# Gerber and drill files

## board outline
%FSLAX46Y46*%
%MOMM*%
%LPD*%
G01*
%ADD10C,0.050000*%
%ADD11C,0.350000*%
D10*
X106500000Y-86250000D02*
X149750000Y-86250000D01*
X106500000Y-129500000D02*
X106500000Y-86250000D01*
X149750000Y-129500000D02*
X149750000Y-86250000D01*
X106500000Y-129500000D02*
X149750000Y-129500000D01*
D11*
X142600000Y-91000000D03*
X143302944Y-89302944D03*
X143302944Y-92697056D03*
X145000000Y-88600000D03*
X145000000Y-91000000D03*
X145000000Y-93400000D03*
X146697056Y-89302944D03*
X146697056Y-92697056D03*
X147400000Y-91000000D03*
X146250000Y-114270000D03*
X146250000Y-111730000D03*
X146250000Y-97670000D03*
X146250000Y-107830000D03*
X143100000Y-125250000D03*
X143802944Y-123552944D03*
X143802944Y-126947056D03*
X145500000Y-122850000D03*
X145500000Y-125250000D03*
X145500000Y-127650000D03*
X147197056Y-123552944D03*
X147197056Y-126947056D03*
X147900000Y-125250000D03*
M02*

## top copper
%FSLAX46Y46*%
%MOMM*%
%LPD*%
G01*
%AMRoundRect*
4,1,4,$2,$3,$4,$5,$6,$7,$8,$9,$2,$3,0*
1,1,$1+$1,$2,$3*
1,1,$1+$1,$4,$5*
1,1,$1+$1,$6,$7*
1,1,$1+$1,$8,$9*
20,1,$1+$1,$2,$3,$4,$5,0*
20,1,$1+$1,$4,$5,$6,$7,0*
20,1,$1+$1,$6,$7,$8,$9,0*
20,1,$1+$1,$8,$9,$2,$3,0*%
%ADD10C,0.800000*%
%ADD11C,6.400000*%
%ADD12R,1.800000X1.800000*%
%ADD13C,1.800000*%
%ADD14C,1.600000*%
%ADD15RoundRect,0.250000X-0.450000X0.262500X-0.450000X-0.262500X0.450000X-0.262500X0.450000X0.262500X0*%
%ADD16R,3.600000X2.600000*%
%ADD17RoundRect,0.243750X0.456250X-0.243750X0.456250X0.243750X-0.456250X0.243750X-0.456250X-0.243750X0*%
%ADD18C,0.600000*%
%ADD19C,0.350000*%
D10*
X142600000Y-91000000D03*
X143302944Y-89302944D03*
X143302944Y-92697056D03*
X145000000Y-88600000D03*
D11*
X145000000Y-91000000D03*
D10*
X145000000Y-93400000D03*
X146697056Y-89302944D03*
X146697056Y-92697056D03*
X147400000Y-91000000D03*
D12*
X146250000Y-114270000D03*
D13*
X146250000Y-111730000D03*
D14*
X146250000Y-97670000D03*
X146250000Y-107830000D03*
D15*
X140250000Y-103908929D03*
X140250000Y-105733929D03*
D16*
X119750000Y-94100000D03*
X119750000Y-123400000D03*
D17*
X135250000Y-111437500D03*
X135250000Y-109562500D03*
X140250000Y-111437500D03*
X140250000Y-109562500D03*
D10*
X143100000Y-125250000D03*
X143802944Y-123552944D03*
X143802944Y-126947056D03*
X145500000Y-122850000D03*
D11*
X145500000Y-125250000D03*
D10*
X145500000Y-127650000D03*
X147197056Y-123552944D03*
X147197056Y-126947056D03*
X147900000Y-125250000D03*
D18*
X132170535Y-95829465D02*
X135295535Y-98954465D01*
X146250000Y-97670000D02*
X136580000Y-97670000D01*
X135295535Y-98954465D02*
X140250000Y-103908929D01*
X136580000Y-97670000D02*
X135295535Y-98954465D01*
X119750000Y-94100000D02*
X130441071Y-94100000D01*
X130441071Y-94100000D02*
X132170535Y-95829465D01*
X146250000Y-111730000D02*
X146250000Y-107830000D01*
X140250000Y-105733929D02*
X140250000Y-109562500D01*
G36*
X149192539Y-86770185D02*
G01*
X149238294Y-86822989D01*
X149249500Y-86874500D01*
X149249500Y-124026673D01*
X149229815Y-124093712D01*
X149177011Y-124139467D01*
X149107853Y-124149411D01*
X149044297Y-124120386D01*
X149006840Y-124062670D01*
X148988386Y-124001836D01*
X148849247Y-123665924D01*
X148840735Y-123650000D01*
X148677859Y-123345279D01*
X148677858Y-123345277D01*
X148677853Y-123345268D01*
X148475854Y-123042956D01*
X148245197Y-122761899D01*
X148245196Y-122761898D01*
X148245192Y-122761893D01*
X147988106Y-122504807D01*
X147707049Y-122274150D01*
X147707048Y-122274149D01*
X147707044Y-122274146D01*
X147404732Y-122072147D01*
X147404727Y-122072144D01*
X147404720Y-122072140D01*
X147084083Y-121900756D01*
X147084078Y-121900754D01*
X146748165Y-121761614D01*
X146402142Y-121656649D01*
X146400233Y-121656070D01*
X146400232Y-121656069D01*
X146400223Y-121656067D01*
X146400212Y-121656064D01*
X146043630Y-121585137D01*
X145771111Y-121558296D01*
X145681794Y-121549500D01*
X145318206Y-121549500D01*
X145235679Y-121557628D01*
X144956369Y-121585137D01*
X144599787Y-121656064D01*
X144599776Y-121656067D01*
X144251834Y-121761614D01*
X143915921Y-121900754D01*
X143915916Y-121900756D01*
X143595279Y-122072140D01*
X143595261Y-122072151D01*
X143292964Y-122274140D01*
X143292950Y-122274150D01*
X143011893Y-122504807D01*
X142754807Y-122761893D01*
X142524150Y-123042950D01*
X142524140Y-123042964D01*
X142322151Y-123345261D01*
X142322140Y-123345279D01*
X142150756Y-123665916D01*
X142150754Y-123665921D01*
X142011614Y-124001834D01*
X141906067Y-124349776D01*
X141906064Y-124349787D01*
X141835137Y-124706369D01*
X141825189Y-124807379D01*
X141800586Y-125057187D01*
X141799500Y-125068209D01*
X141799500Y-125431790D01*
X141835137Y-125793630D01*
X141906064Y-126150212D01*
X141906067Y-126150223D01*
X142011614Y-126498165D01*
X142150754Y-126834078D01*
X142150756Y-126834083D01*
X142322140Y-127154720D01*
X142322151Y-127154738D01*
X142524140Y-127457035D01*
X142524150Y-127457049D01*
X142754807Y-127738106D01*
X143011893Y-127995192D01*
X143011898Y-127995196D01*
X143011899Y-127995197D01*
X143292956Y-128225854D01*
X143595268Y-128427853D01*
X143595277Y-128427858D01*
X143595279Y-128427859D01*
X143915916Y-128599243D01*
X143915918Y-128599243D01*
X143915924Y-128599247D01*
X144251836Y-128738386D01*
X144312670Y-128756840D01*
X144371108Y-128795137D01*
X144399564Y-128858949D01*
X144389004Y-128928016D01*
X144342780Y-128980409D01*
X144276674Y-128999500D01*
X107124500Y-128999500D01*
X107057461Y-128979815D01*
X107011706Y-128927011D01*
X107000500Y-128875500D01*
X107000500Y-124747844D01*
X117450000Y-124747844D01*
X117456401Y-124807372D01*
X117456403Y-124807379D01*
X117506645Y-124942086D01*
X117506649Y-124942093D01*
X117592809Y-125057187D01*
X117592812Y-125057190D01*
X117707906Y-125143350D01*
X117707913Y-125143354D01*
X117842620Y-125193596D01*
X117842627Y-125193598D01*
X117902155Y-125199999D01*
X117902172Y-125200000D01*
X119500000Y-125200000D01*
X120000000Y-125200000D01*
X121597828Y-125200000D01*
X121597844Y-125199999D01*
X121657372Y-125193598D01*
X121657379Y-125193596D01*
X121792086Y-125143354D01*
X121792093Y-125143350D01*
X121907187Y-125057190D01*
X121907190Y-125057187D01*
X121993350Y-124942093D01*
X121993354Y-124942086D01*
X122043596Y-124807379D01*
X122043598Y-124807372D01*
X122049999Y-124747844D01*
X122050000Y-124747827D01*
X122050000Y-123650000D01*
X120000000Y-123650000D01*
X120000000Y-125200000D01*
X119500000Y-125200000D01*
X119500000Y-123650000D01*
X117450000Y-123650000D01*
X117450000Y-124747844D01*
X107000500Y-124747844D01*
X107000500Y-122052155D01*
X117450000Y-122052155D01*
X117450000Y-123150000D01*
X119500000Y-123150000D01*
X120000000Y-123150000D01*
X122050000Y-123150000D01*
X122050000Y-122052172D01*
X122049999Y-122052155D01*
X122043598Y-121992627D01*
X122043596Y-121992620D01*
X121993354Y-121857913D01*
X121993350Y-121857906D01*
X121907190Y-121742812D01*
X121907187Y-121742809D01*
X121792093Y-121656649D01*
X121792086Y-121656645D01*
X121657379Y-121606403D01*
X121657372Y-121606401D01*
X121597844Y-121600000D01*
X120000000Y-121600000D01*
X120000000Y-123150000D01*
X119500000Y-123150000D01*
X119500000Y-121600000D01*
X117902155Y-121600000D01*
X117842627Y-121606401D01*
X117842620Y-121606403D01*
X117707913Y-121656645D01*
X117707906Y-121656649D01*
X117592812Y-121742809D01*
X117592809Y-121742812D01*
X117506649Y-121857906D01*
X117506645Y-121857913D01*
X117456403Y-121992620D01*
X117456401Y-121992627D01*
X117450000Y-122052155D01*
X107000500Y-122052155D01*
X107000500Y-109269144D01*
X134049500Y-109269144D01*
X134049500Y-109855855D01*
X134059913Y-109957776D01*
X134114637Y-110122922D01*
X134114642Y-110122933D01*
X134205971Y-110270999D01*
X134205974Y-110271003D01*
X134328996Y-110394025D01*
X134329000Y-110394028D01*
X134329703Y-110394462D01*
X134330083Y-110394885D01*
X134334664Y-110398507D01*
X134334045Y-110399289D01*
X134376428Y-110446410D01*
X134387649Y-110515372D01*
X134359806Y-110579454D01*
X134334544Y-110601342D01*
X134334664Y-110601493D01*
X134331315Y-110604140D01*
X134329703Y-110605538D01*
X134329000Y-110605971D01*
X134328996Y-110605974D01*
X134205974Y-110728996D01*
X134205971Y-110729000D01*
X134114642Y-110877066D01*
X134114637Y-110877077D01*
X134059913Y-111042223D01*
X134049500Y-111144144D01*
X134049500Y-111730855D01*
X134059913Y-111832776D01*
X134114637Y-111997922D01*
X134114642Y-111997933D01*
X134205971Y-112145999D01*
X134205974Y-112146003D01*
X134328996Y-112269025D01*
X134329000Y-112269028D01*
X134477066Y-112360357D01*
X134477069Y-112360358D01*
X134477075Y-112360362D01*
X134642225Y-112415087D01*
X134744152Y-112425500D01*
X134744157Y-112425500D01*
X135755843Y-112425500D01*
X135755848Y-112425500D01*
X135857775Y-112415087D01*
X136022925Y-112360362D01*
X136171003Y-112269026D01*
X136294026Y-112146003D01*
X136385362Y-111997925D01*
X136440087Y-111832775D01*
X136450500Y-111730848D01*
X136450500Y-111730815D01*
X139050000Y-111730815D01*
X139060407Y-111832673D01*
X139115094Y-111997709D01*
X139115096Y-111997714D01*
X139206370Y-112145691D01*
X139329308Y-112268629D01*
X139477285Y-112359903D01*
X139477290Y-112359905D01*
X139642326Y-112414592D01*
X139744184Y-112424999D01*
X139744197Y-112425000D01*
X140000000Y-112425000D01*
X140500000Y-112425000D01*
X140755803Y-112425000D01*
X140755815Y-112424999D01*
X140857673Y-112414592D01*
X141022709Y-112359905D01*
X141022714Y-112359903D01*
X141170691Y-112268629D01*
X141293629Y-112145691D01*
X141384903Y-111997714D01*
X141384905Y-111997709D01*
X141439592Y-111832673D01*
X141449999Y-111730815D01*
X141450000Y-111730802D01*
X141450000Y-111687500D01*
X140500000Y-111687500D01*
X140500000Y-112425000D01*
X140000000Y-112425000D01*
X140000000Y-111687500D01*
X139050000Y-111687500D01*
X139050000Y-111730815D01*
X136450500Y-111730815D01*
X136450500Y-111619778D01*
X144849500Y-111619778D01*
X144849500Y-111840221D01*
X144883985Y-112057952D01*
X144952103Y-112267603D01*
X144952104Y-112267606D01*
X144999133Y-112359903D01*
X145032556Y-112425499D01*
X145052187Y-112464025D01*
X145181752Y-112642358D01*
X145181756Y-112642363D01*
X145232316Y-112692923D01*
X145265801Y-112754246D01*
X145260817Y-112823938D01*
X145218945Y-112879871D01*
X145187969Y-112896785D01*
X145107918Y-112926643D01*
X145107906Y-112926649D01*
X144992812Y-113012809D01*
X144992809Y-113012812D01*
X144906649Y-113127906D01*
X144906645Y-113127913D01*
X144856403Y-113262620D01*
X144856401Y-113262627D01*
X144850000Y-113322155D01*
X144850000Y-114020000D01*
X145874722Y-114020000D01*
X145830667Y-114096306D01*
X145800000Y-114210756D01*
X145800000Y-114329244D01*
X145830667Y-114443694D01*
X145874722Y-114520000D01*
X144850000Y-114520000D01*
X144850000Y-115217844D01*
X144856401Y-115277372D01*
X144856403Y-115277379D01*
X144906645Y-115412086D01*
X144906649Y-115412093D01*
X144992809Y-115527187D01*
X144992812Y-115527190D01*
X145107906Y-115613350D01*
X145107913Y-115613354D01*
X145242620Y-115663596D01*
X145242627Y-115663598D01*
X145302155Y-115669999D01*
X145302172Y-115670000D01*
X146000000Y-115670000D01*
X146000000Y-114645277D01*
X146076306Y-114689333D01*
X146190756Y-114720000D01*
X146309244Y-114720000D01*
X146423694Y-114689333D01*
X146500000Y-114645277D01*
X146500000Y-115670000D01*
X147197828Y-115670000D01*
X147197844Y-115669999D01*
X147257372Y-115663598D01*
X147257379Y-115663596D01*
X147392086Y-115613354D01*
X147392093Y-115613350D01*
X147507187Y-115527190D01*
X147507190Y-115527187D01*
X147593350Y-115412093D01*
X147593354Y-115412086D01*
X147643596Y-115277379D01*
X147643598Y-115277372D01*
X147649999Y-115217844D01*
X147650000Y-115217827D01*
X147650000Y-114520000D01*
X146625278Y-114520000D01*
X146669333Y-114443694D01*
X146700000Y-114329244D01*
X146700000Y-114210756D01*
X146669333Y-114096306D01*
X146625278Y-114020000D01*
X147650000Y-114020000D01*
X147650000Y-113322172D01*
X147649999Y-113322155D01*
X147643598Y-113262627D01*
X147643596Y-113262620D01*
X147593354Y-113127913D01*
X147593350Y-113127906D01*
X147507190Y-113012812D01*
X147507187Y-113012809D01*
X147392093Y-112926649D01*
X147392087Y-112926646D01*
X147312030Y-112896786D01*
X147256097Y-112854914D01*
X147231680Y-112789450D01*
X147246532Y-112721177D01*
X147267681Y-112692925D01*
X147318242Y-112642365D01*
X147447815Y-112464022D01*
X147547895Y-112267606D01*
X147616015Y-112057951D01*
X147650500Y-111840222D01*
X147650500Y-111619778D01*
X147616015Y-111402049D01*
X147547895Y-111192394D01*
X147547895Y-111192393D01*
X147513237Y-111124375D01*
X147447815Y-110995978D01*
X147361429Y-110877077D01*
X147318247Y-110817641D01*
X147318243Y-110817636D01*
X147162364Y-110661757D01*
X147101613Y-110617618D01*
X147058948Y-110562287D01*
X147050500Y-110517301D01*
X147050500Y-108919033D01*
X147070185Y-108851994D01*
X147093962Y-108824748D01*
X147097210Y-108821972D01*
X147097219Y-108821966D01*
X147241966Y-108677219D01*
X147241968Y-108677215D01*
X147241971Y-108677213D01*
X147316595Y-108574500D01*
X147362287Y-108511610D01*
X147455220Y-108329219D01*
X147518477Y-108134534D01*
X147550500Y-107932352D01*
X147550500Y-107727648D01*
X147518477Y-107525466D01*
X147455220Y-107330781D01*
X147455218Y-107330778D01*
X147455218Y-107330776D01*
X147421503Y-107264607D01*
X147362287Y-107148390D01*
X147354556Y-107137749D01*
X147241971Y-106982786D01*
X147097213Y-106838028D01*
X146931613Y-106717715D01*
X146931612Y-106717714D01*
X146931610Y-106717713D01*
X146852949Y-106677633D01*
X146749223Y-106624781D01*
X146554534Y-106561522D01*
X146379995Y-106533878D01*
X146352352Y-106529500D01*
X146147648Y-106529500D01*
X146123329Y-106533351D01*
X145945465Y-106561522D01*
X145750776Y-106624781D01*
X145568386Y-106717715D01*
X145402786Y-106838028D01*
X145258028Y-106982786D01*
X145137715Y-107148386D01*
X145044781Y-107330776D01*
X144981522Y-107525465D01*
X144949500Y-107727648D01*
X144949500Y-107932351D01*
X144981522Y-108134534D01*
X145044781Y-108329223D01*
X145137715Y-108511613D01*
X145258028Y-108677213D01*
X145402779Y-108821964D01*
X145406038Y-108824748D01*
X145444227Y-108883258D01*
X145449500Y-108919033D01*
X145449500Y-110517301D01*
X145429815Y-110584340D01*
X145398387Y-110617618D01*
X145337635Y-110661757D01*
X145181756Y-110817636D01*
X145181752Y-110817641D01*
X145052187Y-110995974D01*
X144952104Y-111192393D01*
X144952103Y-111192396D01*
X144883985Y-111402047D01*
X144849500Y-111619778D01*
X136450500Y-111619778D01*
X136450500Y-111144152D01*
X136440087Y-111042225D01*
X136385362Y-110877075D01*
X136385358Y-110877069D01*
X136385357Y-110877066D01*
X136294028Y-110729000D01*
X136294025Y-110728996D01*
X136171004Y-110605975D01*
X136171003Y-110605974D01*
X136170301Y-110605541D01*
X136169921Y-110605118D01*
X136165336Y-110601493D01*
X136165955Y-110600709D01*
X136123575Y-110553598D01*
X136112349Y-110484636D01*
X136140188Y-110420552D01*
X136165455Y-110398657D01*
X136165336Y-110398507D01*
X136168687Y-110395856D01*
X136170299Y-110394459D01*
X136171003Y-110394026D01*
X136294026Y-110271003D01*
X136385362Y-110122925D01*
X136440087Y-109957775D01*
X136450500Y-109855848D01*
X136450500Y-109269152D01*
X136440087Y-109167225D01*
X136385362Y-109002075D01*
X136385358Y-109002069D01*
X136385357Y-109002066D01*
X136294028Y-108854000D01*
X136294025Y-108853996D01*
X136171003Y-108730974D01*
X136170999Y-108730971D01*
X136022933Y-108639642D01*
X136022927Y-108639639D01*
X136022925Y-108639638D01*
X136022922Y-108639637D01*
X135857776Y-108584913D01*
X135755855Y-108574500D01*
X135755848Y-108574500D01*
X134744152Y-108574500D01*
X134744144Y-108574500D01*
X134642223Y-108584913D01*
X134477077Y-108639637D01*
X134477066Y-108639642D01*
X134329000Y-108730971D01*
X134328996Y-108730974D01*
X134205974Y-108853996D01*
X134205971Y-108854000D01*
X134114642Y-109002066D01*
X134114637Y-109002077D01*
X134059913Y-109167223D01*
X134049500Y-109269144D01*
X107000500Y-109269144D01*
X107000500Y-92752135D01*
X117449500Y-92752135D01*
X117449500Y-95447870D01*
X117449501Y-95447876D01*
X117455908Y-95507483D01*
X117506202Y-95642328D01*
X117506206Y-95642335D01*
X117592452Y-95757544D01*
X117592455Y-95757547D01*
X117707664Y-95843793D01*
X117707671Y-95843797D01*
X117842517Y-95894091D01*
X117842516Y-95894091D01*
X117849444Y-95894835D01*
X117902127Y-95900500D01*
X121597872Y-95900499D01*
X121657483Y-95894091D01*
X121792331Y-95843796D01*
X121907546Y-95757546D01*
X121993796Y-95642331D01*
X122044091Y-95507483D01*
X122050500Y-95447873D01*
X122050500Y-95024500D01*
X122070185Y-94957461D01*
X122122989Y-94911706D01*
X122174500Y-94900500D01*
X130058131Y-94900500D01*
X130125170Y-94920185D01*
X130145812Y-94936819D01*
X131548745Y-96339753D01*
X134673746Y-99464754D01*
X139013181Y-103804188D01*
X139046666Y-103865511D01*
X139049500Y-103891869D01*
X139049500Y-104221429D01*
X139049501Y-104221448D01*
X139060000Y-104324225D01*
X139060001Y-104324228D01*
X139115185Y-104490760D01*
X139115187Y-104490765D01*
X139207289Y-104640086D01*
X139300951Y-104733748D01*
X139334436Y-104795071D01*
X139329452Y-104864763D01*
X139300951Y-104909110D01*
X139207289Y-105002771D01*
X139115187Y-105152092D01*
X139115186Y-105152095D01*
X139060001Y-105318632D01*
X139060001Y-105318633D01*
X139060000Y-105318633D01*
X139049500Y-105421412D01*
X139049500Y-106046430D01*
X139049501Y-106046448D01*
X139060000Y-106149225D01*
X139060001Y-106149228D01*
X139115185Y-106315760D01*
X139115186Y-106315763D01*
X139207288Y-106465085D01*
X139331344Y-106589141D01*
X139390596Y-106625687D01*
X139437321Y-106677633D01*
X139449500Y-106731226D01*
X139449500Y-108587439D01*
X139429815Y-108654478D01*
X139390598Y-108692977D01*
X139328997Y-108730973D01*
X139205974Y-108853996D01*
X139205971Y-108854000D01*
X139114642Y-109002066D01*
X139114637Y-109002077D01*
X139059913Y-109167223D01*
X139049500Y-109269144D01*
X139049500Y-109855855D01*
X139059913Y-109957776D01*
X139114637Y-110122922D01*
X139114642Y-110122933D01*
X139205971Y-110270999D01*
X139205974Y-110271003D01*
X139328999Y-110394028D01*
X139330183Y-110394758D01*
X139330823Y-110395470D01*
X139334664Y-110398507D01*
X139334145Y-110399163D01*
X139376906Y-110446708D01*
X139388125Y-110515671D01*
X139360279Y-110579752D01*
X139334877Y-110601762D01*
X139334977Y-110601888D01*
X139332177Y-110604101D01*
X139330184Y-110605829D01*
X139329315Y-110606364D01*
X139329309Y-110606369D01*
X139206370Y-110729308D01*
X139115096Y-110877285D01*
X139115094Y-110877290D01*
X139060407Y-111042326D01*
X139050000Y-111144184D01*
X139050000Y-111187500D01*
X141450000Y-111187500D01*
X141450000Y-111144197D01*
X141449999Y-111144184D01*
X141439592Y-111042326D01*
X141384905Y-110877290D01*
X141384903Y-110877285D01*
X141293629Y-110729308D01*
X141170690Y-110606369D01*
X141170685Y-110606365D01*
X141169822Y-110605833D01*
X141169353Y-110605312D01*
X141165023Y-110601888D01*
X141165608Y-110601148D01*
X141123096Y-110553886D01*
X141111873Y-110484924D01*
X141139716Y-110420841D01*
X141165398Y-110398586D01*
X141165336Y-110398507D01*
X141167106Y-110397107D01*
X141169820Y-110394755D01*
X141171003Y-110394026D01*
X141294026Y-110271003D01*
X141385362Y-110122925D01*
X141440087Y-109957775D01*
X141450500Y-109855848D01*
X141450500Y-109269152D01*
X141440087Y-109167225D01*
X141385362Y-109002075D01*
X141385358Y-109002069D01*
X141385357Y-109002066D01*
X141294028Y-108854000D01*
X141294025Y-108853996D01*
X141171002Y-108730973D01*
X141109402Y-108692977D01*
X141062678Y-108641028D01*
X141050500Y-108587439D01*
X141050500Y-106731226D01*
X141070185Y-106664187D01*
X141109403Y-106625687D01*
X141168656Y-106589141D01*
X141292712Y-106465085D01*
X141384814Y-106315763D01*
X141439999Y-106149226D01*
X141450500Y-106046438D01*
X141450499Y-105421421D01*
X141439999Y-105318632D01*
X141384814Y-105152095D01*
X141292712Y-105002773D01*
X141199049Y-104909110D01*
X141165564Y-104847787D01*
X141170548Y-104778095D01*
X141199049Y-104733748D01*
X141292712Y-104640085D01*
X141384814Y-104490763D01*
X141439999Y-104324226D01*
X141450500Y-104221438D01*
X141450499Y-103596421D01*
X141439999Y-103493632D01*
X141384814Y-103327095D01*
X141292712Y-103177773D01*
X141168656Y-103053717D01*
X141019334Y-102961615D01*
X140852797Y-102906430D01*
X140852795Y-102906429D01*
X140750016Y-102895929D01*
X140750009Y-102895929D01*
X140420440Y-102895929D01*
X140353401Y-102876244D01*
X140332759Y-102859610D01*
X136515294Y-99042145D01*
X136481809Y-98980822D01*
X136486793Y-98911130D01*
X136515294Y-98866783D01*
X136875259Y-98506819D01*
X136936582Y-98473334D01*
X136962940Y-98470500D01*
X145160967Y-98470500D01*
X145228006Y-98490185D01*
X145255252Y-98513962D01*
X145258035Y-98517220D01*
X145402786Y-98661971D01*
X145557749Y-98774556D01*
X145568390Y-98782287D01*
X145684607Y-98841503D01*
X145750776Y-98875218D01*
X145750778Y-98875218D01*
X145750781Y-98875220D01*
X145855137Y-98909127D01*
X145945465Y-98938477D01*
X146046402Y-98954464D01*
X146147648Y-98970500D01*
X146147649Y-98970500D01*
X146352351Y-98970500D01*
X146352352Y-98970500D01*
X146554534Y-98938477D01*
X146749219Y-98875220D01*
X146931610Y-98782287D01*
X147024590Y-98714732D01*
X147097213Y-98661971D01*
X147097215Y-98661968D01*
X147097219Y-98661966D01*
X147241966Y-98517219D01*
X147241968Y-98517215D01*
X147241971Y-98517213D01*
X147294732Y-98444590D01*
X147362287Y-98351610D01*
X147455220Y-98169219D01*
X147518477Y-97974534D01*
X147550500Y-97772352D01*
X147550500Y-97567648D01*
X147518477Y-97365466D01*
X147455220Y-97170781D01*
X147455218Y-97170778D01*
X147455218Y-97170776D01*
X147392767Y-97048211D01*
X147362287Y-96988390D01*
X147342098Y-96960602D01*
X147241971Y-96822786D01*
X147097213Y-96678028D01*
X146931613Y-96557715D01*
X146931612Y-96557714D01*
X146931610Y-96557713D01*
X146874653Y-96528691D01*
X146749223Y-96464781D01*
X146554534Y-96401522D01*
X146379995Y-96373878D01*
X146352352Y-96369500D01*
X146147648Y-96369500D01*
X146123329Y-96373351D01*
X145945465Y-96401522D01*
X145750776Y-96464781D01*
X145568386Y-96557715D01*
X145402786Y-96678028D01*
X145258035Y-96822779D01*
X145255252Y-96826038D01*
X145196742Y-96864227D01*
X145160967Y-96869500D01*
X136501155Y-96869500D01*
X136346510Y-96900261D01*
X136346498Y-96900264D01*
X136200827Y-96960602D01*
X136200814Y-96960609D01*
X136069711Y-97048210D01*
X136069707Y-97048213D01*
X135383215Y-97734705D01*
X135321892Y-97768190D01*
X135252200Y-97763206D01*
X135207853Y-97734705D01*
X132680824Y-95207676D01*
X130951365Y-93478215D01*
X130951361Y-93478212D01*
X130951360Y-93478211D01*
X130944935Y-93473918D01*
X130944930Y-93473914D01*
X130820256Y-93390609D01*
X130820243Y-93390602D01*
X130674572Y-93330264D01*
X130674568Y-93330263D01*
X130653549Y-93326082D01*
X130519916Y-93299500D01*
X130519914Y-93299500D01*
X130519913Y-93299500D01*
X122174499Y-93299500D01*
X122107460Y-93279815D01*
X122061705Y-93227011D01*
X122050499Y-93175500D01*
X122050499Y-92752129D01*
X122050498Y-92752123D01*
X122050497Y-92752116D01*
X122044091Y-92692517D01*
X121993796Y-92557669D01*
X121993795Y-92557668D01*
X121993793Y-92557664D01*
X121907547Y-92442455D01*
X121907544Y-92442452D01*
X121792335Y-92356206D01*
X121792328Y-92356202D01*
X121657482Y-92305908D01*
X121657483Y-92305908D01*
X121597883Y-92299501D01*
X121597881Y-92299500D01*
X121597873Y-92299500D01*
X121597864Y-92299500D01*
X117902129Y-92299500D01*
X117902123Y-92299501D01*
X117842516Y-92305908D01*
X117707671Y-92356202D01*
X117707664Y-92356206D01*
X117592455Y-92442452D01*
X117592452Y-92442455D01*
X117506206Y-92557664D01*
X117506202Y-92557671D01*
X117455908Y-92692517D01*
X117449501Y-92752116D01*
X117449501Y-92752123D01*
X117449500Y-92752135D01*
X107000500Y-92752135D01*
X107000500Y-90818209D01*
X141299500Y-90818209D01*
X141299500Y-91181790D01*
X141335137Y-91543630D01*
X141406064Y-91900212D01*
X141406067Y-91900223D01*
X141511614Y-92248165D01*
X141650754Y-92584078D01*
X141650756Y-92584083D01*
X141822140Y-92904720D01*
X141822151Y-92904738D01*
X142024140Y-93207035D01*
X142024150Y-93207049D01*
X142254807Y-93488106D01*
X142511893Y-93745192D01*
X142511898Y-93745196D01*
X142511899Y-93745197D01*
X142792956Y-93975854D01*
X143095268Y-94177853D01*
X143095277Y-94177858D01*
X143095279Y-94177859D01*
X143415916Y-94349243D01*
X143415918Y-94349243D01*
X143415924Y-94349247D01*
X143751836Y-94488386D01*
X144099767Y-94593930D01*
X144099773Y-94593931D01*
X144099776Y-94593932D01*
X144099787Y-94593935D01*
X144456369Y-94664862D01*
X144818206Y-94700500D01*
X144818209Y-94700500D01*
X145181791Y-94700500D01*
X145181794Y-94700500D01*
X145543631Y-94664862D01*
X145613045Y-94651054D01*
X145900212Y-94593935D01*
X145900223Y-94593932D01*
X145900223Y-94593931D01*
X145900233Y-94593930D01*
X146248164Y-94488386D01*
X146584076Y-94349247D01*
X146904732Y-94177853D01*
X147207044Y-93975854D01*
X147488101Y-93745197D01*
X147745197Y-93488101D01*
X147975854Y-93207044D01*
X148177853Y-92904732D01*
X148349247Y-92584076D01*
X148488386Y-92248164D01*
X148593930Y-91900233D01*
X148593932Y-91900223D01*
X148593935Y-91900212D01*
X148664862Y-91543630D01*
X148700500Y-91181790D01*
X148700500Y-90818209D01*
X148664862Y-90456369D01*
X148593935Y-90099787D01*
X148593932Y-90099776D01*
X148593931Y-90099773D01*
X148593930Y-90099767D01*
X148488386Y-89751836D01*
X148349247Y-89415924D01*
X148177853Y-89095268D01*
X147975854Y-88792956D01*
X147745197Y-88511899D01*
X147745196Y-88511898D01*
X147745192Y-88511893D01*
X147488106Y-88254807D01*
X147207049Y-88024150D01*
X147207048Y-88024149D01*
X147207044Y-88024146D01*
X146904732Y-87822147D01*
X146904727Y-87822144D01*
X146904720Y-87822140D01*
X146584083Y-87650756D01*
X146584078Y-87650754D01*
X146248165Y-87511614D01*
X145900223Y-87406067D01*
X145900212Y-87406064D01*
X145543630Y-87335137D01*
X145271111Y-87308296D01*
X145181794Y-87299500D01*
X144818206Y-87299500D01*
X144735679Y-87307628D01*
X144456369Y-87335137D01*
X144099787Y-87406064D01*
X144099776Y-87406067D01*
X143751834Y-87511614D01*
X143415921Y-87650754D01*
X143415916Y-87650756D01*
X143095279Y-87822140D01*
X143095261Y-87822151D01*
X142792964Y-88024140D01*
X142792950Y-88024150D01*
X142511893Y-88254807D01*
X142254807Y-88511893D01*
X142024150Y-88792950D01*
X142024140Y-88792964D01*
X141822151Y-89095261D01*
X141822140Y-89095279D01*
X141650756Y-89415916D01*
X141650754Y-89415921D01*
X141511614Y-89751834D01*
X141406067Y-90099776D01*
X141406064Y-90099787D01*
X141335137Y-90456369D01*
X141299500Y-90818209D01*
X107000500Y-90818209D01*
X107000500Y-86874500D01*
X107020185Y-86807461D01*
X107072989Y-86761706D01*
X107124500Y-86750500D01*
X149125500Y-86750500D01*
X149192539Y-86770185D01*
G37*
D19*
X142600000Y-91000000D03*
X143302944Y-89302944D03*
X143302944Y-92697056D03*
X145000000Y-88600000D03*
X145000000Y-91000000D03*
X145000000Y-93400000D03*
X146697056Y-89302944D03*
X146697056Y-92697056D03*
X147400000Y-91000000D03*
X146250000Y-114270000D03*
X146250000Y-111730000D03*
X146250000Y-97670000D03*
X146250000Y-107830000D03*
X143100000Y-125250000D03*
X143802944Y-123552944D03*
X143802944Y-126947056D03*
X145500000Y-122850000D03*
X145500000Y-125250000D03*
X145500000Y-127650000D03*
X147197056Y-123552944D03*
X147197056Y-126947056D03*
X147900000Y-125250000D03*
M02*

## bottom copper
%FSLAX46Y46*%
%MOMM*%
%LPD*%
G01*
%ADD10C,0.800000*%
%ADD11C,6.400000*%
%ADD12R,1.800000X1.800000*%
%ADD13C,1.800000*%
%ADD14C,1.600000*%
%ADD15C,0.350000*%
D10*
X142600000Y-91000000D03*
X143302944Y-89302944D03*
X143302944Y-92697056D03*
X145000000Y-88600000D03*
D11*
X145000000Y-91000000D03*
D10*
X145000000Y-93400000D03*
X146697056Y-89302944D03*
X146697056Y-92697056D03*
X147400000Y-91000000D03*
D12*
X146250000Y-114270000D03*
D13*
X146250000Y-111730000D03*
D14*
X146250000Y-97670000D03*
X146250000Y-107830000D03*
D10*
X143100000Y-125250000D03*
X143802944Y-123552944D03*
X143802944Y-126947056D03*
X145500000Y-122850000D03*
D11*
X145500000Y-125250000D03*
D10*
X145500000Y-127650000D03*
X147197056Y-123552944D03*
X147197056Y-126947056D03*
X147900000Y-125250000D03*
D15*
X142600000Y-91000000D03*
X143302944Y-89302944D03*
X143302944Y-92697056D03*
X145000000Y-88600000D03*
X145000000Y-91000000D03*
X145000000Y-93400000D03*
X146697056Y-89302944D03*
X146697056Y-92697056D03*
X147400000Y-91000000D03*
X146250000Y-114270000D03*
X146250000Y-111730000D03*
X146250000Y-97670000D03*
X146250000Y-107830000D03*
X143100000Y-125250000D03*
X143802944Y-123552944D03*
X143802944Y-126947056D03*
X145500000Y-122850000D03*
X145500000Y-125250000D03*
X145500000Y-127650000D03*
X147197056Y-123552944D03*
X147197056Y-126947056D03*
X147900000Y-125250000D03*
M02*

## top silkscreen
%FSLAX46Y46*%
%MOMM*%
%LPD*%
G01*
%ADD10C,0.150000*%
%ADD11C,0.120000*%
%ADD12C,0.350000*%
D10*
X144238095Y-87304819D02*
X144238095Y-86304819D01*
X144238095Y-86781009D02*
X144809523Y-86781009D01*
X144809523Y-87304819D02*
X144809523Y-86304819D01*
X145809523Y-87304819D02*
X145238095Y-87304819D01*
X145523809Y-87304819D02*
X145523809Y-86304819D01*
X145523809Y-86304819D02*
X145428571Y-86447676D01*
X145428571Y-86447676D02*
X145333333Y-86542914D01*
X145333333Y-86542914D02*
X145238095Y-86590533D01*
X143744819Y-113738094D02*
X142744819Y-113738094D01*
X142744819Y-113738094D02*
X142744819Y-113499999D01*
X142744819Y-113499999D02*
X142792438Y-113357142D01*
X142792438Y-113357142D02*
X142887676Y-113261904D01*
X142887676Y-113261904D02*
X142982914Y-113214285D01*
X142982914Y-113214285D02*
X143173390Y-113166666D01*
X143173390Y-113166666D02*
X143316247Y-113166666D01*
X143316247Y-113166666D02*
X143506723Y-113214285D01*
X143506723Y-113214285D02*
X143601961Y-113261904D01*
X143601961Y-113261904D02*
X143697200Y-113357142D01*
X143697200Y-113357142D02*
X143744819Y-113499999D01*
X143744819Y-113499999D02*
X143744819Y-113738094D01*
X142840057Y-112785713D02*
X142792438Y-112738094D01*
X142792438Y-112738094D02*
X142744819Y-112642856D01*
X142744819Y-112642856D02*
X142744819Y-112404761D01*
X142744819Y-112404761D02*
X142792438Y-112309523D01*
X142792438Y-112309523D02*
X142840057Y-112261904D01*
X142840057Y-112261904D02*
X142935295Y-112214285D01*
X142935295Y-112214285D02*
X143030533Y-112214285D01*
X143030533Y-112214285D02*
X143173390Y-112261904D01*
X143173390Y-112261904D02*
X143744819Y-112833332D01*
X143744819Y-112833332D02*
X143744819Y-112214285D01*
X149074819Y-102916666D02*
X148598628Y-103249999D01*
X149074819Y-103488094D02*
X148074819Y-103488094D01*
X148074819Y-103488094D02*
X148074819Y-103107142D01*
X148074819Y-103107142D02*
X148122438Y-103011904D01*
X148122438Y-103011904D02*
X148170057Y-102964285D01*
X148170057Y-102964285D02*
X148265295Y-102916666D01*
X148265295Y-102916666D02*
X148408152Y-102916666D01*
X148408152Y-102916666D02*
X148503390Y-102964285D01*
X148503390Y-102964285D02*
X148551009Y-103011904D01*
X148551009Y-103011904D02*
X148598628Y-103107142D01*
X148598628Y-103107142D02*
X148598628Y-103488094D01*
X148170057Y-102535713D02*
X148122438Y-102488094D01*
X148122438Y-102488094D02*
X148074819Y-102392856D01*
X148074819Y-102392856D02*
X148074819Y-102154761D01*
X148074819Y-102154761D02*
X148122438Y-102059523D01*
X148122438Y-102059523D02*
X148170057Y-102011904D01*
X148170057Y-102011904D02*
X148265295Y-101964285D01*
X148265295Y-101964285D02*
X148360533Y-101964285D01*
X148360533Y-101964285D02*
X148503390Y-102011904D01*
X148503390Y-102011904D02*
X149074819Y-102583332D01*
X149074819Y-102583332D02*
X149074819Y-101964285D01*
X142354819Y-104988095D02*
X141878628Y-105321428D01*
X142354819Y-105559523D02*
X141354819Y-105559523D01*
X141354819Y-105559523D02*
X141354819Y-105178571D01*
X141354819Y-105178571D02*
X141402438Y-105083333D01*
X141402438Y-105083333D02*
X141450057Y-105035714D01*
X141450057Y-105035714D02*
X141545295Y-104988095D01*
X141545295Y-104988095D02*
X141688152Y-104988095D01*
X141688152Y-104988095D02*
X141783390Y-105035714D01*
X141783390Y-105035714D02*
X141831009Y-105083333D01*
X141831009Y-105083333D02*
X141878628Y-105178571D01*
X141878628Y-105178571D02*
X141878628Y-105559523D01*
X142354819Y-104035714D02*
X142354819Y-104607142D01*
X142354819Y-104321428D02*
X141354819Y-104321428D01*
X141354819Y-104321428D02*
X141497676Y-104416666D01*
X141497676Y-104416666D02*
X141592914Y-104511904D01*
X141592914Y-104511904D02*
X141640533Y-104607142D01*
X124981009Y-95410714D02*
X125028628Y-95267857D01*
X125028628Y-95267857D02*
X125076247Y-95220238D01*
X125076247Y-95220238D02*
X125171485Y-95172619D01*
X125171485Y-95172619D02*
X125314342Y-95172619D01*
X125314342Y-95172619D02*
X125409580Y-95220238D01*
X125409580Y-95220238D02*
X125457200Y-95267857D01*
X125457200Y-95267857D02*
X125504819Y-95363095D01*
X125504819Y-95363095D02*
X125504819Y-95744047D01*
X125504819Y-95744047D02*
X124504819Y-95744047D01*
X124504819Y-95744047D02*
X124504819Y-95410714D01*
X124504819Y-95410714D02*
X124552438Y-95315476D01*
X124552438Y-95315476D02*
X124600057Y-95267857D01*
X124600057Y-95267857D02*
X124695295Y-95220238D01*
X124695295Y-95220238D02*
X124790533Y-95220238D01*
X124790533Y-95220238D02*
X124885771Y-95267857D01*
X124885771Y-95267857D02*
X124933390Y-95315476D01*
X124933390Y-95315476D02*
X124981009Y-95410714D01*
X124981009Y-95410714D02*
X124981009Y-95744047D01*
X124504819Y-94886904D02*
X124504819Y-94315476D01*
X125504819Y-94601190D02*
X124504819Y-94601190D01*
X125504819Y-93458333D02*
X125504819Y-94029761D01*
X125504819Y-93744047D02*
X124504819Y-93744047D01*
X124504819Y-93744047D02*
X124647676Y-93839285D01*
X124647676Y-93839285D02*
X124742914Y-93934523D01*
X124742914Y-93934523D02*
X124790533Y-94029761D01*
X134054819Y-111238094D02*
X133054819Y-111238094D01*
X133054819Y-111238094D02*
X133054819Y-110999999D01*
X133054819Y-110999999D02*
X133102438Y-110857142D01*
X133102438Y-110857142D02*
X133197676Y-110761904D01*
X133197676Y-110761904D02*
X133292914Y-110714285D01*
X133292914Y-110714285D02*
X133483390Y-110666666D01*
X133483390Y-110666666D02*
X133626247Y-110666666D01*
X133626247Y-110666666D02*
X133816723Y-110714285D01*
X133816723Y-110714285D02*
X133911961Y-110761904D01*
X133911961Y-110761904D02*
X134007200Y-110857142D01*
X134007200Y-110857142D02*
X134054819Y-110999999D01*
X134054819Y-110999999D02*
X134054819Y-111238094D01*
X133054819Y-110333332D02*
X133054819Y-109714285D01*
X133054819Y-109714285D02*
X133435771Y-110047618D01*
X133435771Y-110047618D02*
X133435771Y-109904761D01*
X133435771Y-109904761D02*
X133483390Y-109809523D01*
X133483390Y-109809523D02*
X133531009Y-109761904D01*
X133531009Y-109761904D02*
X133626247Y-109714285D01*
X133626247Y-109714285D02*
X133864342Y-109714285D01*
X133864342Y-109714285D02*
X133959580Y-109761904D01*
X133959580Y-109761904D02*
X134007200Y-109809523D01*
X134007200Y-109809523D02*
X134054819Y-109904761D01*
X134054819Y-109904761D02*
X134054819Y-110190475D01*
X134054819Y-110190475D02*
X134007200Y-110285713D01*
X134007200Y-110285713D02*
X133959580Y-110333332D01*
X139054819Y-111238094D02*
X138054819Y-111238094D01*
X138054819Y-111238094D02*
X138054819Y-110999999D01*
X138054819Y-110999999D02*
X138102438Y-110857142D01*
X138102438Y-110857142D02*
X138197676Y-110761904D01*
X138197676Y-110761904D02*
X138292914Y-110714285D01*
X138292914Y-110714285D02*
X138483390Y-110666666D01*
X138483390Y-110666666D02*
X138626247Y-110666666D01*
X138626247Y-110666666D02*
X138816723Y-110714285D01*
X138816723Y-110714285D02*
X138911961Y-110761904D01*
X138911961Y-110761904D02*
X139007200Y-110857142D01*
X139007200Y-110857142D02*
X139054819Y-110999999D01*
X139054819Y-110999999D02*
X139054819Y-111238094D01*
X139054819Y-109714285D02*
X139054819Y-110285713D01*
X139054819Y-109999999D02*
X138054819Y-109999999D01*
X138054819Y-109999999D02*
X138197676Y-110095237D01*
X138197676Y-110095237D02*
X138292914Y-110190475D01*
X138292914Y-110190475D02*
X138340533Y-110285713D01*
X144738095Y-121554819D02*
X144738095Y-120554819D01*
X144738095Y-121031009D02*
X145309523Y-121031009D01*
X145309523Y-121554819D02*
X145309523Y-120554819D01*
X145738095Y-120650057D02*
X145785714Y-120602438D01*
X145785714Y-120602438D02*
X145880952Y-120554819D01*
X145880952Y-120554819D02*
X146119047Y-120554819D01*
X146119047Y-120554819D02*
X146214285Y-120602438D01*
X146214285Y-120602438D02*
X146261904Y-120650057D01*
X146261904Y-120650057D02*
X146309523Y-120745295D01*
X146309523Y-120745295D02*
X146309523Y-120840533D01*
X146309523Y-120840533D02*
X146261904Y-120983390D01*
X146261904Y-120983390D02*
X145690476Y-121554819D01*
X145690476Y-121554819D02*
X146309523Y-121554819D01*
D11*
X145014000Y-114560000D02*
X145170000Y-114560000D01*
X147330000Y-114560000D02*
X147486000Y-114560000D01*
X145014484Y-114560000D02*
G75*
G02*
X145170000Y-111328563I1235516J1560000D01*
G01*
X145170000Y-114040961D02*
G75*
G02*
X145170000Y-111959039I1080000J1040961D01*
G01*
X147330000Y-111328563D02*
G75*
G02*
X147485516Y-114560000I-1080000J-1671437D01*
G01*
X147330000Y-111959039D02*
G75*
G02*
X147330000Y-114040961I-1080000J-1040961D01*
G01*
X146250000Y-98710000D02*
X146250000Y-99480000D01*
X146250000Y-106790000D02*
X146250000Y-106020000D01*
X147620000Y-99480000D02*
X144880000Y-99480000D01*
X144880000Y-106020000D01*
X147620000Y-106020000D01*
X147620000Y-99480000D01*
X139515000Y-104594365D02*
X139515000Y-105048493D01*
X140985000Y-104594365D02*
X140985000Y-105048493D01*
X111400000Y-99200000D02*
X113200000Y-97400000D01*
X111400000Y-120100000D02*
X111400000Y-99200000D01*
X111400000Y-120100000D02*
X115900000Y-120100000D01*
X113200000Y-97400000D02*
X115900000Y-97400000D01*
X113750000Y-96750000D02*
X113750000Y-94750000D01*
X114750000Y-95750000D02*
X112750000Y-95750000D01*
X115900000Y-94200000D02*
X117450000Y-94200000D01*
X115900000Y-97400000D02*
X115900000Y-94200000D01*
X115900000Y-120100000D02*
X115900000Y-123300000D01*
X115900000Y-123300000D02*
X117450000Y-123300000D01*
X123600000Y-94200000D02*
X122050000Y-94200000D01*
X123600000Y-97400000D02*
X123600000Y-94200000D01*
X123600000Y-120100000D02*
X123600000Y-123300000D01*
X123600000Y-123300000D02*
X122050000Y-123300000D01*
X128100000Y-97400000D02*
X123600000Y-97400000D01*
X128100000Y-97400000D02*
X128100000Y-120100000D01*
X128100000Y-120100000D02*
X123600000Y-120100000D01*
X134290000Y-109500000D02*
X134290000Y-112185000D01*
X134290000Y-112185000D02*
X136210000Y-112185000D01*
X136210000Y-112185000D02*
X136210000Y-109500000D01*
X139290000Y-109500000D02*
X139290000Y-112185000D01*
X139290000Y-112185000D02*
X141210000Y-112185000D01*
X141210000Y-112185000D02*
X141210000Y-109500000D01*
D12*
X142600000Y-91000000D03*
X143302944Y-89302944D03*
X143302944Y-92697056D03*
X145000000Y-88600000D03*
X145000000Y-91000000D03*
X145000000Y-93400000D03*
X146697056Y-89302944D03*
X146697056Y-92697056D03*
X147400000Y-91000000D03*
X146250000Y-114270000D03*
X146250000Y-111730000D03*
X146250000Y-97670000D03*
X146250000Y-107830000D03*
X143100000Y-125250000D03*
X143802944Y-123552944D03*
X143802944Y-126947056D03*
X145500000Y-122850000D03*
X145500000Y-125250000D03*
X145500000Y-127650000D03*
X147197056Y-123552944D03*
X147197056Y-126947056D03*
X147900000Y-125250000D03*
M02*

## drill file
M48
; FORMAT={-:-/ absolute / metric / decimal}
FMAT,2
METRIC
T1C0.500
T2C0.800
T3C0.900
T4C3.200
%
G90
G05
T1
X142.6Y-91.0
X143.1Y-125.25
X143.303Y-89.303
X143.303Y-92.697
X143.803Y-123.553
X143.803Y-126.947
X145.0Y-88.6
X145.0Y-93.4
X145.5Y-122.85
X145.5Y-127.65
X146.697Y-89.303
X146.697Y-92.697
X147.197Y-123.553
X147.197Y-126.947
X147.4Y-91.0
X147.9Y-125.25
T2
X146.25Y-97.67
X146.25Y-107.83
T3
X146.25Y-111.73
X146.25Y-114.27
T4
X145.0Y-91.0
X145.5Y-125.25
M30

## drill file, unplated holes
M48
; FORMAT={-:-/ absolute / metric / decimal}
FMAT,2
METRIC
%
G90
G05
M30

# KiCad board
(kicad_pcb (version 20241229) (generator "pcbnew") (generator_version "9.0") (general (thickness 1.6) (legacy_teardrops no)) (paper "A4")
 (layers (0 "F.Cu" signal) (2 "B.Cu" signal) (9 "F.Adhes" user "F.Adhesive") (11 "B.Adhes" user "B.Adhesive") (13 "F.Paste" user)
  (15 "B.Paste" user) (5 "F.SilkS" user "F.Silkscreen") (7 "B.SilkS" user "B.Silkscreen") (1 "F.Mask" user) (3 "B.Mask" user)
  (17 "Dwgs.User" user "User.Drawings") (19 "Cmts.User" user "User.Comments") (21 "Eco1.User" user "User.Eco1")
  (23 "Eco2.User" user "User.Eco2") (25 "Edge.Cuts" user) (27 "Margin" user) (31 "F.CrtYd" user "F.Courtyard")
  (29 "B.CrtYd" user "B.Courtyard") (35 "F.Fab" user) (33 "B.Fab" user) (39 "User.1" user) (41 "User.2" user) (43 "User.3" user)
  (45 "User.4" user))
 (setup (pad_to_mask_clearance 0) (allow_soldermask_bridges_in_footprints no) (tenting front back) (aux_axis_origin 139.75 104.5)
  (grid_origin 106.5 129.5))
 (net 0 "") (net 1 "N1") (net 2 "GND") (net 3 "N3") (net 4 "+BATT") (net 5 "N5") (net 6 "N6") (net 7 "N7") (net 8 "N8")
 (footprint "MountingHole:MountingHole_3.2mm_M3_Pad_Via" (layer "F.Cu") (at 145 91)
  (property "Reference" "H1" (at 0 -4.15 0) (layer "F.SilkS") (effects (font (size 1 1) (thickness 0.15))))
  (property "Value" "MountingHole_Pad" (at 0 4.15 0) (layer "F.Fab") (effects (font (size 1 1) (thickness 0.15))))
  (pad "1" thru_hole circle (at -2.4 0) (size 0.8 0.8) (drill 0.5) (layers "*.Cu" "*.Mask") (remove_unused_layers no) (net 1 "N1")
   (zone_connect 2))
  (pad "1" thru_hole circle (at -1.697056 -1.697056) (size 0.8 0.8) (drill 0.5) (layers "*.Cu" "*.Mask") (remove_unused_layers no)
   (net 1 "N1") (zone_connect 2))
  (pad "1" thru_hole circle (at -1.697056 1.697056) (size 0.8 0.8) (drill 0.5) (layers "*.Cu" "*.Mask") (remove_unused_layers no)
   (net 1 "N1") (zone_connect 2))
  (pad "1" thru_hole circle (at 0 -2.4) (size 0.8 0.8) (drill 0.5) (layers "*.Cu" "*.Mask") (remove_unused_layers no) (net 1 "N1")
   (zone_connect 2))
  (pad "1" thru_hole circle (at 0 0) (size 6.4 6.4) (drill 3.2) (layers "*.Cu" "*.Mask") (remove_unused_layers no) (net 1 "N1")
   (zone_connect 2))
  (pad "1" thru_hole circle (at 0 2.4) (size 0.8 0.8) (drill 0.5) (layers "*.Cu" "*.Mask") (remove_unused_layers no) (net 1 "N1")
   (zone_connect 2))
  (pad "1" thru_hole circle (at 1.697056 -1.697056) (size 0.8 0.8) (drill 0.5) (layers "*.Cu" "*.Mask") (remove_unused_layers no)
   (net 1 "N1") (zone_connect 2))
  (pad "1" thru_hole circle (at 1.697056 1.697056) (size 0.8 0.8) (drill 0.5) (layers "*.Cu" "*.Mask") (remove_unused_layers no)
   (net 1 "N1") (zone_connect 2))
  (pad "1" thru_hole circle (at 2.4 0) (size 0.8 0.8) (drill 0.5) (layers "*.Cu" "*.Mask") (remove_unused_layers no) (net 1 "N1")
   (zone_connect 2)))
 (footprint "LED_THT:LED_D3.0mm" (layer "F.Cu") (at 146.25 114.27 90)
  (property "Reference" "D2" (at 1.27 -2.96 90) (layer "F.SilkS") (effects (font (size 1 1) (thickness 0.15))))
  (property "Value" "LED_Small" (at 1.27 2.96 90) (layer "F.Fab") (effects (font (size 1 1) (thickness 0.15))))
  (fp_line (start -0.29 -1.236) (end -0.29 -1.08) (stroke (width 0.12) (type solid)) (layer "F.SilkS"))
  (fp_line (start -0.29 1.08) (end -0.29 1.236) (stroke (width 0.12) (type solid)) (layer "F.SilkS"))
  (fp_arc (start -0.29 -1.235516) (mid 1.36566 -1.987699) (end 2.941437 -1.08) (stroke (width 0.12) (type solid)) (layer "F.SilkS"))
  (fp_arc (start 0.229039 -1.08) (mid 1.27 -1.5) (end 2.310961 -1.08) (stroke (width 0.12) (type solid)) (layer "F.SilkS"))
  (fp_arc (start 2.941437 1.08) (mid 1.36566 1.987699) (end -0.29 1.235516) (stroke (width 0.12) (type solid)) (layer "F.SilkS"))
  (fp_arc (start 2.310961 1.08) (mid 1.27 1.5) (end 0.229039 1.08) (stroke (width 0.12) (type solid)) (layer "F.SilkS"))
  (pad "1" thru_hole rect (at 0 0 90) (size 1.8 1.8) (drill 0.9) (layers "*.Cu" "*.Mask") (remove_unused_layers no) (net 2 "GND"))
  (pad "2" thru_hole circle (at 2.54 0 90) (size 1.8 1.8) (drill 0.9) (layers "*.Cu" "*.Mask") (remove_unused_layers no) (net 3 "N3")))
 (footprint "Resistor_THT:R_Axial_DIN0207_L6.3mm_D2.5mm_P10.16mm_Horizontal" (layer "F.Cu") (at 146.25 97.67 -90)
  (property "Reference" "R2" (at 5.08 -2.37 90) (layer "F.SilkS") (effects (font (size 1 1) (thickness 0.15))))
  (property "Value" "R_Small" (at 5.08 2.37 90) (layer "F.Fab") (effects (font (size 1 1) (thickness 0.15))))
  (fp_line (start 1.04 0) (end 1.81 0) (stroke (width 0.12) (type solid)) (layer "F.SilkS"))
  (fp_line (start 9.12 0) (end 8.35 0) (stroke (width 0.12) (type solid)) (layer "F.SilkS"))
  (fp_rect (start 1.81 -1.37) (end 8.35 1.37) (stroke (width 0.12) (type solid)) (fill no) (layer "F.SilkS"))
  (pad "1" thru_hole circle (at 0 0 270) (size 1.6 1.6) (drill 0.8) (layers "*.Cu" "*.Mask") (remove_unused_layers no) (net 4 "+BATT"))
  (pad "2" thru_hole circle (at 10.16 0 270) (size 1.6 1.6) (drill 0.8) (layers "*.Cu" "*.Mask") (remove_unused_layers no) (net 3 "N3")))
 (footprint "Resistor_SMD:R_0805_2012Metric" (layer "F.Cu") (at 140.25 104.821429 -90)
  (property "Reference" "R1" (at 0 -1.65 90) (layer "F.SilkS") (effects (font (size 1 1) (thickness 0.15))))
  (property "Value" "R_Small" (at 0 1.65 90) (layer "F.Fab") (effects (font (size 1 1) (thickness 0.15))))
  (fp_line (start -0.227064 0.735) (end 0.227064 0.735) (stroke (width 0.12) (type solid)) (layer "F.SilkS"))
  (fp_line (start -0.227064 -0.735) (end 0.227064 -0.735) (stroke (width 0.12) (type solid)) (layer "F.SilkS"))
  (pad "1" smd roundrect (at -0.9125 0 270) (size 1.025 1.4) (layers "F.Cu" "F.Mask" "F.Paste") (roundrect_rratio 0.243902) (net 4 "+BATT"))
  (pad "2" smd roundrect (at 0.9125 0 270) (size 1.025 1.4) (layers "F.Cu" "F.Mask" "F.Paste") (roundrect_rratio 0.243902) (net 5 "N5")))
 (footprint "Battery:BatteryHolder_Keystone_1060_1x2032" (layer "F.Cu") (at 119.75 108.75 -90)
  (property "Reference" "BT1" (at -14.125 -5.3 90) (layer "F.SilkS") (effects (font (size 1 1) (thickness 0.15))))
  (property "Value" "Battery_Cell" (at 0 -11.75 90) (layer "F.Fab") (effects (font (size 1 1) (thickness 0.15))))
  (fp_line (start -9.55 8.35) (end -11.35 6.55) (stroke (width 0.12) (type solid)) (layer "F.SilkS"))
  (fp_line (start 11.35 8.35) (end -9.55 8.35) (stroke (width 0.12) (type solid)) (layer "F.SilkS"))
  (fp_line (start 11.35 8.35) (end 11.35 3.85) (stroke (width 0.12) (type solid)) (layer "F.SilkS"))
  (fp_line (start -11.35 6.55) (end -11.35 3.85) (stroke (width 0.12) (type solid)) (layer "F.SilkS"))
  (fp_line (start -12 6) (end -14 6) (stroke (width 0.12) (type solid)) (layer "F.SilkS"))
  (fp_line (start -13 5) (end -13 7) (stroke (width 0.12) (type solid)) (layer "F.SilkS"))
  (fp_line (start -14.55 3.85) (end -14.55 2.3) (stroke (width 0.12) (type solid)) (layer "F.SilkS"))
  (fp_line (start -11.35 3.85) (end -14.55 3.85) (stroke (width 0.12) (type solid)) (layer "F.SilkS"))
  (fp_line (start 11.35 3.85) (end 14.55 3.85) (stroke (width 0.12) (type solid)) (layer "F.SilkS"))
  (fp_line (start 14.55 3.85) (end 14.55 2.3) (stroke (width 0.12) (type solid)) (layer "F.SilkS"))
  (fp_line (start -14.55 -3.85) (end -14.55 -2.3) (stroke (width 0.12) (type solid)) (layer "F.SilkS"))
  (fp_line (start -11.35 -3.85) (end -14.55 -3.85) (stroke (width 0.12) (type solid)) (layer "F.SilkS"))
  (fp_line (start 11.35 -3.85) (end 14.55 -3.85) (stroke (width 0.12) (type solid)) (layer "F.SilkS"))
  (fp_line (start 14.55 -3.85) (end 14.55 -2.3) (stroke (width 0.12) (type solid)) (layer "F.SilkS"))
  (fp_line (start -11.35 -8.35) (end -11.35 -3.85) (stroke (width 0.12) (type solid)) (layer "F.SilkS"))
  (fp_line (start -11.35 -8.35) (end 11.35 -8.35) (stroke (width 0.12) (type solid)) (layer "F.SilkS"))
  (fp_line (start 11.35 -8.35) (end 11.35 -3.85) (stroke (width 0.12) (type solid)) (layer "F.SilkS"))
  (pad "1" smd rect (at -14.65 0 90) (size 2.6 3.6) (layers "F.Cu" "F.Mask" "F.Paste") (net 4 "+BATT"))
  (pad "2" smd rect (at 14.65 0 90) (size 2.6 3.6) (layers "F.Cu" "F.Mask" "F.Paste") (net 2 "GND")))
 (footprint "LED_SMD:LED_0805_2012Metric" (layer "F.Cu") (at 135.25 110.5 90)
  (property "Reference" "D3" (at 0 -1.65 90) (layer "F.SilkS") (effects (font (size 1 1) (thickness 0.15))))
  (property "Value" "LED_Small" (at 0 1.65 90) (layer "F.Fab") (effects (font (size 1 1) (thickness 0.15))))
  (fp_line (start 1 -0.96) (end -1.685 -0.96) (stroke (width 0.12) (type solid)) (layer "F.SilkS"))
  (fp_line (start -1.685 -0.96) (end -1.685 0.96) (stroke (width 0.12) (type solid)) (layer "F.SilkS"))
  (fp_line (start -1.685 0.96) (end 1 0.96) (stroke (width 0.12) (type solid)) (layer "F.SilkS"))
  (pad "1" smd roundrect (at -0.9375 0 90) (size 0.975 1.4) (layers "F.Cu" "F.Mask" "F.Paste") (roundrect_rratio 0.25) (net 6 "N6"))
  (pad "2" smd roundrect (at 0.9375 0 90) (size 0.975 1.4) (layers "F.Cu" "F.Mask" "F.Paste") (roundrect_rratio 0.25) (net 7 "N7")))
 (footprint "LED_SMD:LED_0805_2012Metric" (layer "F.Cu") (at 140.25 110.5 90)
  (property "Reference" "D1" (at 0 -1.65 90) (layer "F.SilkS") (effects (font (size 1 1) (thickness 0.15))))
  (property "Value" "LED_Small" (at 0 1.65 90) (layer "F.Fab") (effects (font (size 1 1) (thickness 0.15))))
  (fp_line (start 1 -0.96) (end -1.685 -0.96) (stroke (width 0.12) (type solid)) (layer "F.SilkS"))
  (fp_line (start -1.685 -0.96) (end -1.685 0.96) (stroke (width 0.12) (type solid)) (layer "F.SilkS"))
  (fp_line (start -1.685 0.96) (end 1 0.96) (stroke (width 0.12) (type solid)) (layer "F.SilkS"))
  (pad "1" smd roundrect (at -0.9375 0 90) (size 0.975 1.4) (layers "F.Cu" "F.Mask" "F.Paste") (roundrect_rratio 0.25) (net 2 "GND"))
  (pad "2" smd roundrect (at 0.9375 0 90) (size 0.975 1.4) (layers "F.Cu" "F.Mask" "F.Paste") (roundrect_rratio 0.25) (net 5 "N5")))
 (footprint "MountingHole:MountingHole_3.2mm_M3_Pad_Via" (layer "F.Cu") (at 145.5 125.25)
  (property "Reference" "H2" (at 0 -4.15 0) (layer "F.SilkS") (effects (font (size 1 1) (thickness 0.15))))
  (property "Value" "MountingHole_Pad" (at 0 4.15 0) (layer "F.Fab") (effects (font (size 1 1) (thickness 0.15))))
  (pad "1" thru_hole circle (at -2.4 0) (size 0.8 0.8) (drill 0.5) (layers "*.Cu" "*.Mask") (remove_unused_layers no) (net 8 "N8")
   (zone_connect 2))
  (pad "1" thru_hole circle (at -1.697056 -1.697056) (size 0.8 0.8) (drill 0.5) (layers "*.Cu" "*.Mask") (remove_unused_layers no)
   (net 8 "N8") (zone_connect 2))
  (pad "1" thru_hole circle (at -1.697056 1.697056) (size 0.8 0.8) (drill 0.5) (layers "*.Cu" "*.Mask") (remove_unused_layers no)
   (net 8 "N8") (zone_connect 2))
  (pad "1" thru_hole circle (at 0 -2.4) (size 0.8 0.8) (drill 0.5) (layers "*.Cu" "*.Mask") (remove_unused_layers no) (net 8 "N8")
   (zone_connect 2))
  (pad "1" thru_hole circle (at 0 0) (size 6.4 6.4) (drill 3.2) (layers "*.Cu" "*.Mask") (remove_unused_layers no) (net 8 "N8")
   (zone_connect 2))
  (pad "1" thru_hole circle (at 0 2.4) (size 0.8 0.8) (drill 0.5) (layers "*.Cu" "*.Mask") (remove_unused_layers no) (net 8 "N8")
   (zone_connect 2))
  (pad "1" thru_hole circle (at 1.697056 -1.697056) (size 0.8 0.8) (drill 0.5) (layers "*.Cu" "*.Mask") (remove_unused_layers no)
   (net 8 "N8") (zone_connect 2))
  (pad "1" thru_hole circle (at 1.697056 1.697056) (size 0.8 0.8) (drill 0.5) (layers "*.Cu" "*.Mask") (remove_unused_layers no)
   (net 8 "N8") (zone_connect 2))
  (pad "1" thru_hole circle (at 2.4 0) (size 0.8 0.8) (drill 0.5) (layers "*.Cu" "*.Mask") (remove_unused_layers no) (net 8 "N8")
   (zone_connect 2)))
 (gr_line (start 106.5 86.25) (end 149.75 86.25) (stroke (width 0.05) (type default)) (layer "Edge.Cuts"))
 (gr_line (start 106.5 129.5) (end 106.5 86.25) (stroke (width 0.05) (type default)) (layer "Edge.Cuts"))
 (gr_line (start 149.75 129.5) (end 149.75 86.25) (stroke (width 0.05) (type default)) (layer "Edge.Cuts"))
 (gr_line (start 106.5 129.5) (end 149.75 129.5) (stroke (width 0.05) (type default)) (layer "Edge.Cuts"))
 (segment (start 132.170535 95.829465) (end 135.295535 98.954465) (width 0.6) (layer "F.Cu") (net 4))
 (segment (start 146.25 97.67) (end 136.58 97.67) (width 0.6) (layer "F.Cu") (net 4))
 (segment (start 135.295535 98.954465) (end 140.25 103.908929) (width 0.6) (layer "F.Cu") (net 4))
 (segment (start 136.58 97.67) (end 135.295535 98.954465) (width 0.6) (layer "F.Cu") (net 4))
 (segment (start 119.75 94.1) (end 130.441071 94.1) (width 0.6) (layer "F.Cu") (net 4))
 (segment (start 130.441071 94.1) (end 132.170535 95.829465) (width 0.6) (layer "F.Cu") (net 4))
 (segment (start 146.25 111.73) (end 146.25 107.83) (width 0.6) (layer "F.Cu") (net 3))
 (segment (start 140.25 105.733929) (end 140.25 109.5625) (width 0.6) (layer "F.Cu") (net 5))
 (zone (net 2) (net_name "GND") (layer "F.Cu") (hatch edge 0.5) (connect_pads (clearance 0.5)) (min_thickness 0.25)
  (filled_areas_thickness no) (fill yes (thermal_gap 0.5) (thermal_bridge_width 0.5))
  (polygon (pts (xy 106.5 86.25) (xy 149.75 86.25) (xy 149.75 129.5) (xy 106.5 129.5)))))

